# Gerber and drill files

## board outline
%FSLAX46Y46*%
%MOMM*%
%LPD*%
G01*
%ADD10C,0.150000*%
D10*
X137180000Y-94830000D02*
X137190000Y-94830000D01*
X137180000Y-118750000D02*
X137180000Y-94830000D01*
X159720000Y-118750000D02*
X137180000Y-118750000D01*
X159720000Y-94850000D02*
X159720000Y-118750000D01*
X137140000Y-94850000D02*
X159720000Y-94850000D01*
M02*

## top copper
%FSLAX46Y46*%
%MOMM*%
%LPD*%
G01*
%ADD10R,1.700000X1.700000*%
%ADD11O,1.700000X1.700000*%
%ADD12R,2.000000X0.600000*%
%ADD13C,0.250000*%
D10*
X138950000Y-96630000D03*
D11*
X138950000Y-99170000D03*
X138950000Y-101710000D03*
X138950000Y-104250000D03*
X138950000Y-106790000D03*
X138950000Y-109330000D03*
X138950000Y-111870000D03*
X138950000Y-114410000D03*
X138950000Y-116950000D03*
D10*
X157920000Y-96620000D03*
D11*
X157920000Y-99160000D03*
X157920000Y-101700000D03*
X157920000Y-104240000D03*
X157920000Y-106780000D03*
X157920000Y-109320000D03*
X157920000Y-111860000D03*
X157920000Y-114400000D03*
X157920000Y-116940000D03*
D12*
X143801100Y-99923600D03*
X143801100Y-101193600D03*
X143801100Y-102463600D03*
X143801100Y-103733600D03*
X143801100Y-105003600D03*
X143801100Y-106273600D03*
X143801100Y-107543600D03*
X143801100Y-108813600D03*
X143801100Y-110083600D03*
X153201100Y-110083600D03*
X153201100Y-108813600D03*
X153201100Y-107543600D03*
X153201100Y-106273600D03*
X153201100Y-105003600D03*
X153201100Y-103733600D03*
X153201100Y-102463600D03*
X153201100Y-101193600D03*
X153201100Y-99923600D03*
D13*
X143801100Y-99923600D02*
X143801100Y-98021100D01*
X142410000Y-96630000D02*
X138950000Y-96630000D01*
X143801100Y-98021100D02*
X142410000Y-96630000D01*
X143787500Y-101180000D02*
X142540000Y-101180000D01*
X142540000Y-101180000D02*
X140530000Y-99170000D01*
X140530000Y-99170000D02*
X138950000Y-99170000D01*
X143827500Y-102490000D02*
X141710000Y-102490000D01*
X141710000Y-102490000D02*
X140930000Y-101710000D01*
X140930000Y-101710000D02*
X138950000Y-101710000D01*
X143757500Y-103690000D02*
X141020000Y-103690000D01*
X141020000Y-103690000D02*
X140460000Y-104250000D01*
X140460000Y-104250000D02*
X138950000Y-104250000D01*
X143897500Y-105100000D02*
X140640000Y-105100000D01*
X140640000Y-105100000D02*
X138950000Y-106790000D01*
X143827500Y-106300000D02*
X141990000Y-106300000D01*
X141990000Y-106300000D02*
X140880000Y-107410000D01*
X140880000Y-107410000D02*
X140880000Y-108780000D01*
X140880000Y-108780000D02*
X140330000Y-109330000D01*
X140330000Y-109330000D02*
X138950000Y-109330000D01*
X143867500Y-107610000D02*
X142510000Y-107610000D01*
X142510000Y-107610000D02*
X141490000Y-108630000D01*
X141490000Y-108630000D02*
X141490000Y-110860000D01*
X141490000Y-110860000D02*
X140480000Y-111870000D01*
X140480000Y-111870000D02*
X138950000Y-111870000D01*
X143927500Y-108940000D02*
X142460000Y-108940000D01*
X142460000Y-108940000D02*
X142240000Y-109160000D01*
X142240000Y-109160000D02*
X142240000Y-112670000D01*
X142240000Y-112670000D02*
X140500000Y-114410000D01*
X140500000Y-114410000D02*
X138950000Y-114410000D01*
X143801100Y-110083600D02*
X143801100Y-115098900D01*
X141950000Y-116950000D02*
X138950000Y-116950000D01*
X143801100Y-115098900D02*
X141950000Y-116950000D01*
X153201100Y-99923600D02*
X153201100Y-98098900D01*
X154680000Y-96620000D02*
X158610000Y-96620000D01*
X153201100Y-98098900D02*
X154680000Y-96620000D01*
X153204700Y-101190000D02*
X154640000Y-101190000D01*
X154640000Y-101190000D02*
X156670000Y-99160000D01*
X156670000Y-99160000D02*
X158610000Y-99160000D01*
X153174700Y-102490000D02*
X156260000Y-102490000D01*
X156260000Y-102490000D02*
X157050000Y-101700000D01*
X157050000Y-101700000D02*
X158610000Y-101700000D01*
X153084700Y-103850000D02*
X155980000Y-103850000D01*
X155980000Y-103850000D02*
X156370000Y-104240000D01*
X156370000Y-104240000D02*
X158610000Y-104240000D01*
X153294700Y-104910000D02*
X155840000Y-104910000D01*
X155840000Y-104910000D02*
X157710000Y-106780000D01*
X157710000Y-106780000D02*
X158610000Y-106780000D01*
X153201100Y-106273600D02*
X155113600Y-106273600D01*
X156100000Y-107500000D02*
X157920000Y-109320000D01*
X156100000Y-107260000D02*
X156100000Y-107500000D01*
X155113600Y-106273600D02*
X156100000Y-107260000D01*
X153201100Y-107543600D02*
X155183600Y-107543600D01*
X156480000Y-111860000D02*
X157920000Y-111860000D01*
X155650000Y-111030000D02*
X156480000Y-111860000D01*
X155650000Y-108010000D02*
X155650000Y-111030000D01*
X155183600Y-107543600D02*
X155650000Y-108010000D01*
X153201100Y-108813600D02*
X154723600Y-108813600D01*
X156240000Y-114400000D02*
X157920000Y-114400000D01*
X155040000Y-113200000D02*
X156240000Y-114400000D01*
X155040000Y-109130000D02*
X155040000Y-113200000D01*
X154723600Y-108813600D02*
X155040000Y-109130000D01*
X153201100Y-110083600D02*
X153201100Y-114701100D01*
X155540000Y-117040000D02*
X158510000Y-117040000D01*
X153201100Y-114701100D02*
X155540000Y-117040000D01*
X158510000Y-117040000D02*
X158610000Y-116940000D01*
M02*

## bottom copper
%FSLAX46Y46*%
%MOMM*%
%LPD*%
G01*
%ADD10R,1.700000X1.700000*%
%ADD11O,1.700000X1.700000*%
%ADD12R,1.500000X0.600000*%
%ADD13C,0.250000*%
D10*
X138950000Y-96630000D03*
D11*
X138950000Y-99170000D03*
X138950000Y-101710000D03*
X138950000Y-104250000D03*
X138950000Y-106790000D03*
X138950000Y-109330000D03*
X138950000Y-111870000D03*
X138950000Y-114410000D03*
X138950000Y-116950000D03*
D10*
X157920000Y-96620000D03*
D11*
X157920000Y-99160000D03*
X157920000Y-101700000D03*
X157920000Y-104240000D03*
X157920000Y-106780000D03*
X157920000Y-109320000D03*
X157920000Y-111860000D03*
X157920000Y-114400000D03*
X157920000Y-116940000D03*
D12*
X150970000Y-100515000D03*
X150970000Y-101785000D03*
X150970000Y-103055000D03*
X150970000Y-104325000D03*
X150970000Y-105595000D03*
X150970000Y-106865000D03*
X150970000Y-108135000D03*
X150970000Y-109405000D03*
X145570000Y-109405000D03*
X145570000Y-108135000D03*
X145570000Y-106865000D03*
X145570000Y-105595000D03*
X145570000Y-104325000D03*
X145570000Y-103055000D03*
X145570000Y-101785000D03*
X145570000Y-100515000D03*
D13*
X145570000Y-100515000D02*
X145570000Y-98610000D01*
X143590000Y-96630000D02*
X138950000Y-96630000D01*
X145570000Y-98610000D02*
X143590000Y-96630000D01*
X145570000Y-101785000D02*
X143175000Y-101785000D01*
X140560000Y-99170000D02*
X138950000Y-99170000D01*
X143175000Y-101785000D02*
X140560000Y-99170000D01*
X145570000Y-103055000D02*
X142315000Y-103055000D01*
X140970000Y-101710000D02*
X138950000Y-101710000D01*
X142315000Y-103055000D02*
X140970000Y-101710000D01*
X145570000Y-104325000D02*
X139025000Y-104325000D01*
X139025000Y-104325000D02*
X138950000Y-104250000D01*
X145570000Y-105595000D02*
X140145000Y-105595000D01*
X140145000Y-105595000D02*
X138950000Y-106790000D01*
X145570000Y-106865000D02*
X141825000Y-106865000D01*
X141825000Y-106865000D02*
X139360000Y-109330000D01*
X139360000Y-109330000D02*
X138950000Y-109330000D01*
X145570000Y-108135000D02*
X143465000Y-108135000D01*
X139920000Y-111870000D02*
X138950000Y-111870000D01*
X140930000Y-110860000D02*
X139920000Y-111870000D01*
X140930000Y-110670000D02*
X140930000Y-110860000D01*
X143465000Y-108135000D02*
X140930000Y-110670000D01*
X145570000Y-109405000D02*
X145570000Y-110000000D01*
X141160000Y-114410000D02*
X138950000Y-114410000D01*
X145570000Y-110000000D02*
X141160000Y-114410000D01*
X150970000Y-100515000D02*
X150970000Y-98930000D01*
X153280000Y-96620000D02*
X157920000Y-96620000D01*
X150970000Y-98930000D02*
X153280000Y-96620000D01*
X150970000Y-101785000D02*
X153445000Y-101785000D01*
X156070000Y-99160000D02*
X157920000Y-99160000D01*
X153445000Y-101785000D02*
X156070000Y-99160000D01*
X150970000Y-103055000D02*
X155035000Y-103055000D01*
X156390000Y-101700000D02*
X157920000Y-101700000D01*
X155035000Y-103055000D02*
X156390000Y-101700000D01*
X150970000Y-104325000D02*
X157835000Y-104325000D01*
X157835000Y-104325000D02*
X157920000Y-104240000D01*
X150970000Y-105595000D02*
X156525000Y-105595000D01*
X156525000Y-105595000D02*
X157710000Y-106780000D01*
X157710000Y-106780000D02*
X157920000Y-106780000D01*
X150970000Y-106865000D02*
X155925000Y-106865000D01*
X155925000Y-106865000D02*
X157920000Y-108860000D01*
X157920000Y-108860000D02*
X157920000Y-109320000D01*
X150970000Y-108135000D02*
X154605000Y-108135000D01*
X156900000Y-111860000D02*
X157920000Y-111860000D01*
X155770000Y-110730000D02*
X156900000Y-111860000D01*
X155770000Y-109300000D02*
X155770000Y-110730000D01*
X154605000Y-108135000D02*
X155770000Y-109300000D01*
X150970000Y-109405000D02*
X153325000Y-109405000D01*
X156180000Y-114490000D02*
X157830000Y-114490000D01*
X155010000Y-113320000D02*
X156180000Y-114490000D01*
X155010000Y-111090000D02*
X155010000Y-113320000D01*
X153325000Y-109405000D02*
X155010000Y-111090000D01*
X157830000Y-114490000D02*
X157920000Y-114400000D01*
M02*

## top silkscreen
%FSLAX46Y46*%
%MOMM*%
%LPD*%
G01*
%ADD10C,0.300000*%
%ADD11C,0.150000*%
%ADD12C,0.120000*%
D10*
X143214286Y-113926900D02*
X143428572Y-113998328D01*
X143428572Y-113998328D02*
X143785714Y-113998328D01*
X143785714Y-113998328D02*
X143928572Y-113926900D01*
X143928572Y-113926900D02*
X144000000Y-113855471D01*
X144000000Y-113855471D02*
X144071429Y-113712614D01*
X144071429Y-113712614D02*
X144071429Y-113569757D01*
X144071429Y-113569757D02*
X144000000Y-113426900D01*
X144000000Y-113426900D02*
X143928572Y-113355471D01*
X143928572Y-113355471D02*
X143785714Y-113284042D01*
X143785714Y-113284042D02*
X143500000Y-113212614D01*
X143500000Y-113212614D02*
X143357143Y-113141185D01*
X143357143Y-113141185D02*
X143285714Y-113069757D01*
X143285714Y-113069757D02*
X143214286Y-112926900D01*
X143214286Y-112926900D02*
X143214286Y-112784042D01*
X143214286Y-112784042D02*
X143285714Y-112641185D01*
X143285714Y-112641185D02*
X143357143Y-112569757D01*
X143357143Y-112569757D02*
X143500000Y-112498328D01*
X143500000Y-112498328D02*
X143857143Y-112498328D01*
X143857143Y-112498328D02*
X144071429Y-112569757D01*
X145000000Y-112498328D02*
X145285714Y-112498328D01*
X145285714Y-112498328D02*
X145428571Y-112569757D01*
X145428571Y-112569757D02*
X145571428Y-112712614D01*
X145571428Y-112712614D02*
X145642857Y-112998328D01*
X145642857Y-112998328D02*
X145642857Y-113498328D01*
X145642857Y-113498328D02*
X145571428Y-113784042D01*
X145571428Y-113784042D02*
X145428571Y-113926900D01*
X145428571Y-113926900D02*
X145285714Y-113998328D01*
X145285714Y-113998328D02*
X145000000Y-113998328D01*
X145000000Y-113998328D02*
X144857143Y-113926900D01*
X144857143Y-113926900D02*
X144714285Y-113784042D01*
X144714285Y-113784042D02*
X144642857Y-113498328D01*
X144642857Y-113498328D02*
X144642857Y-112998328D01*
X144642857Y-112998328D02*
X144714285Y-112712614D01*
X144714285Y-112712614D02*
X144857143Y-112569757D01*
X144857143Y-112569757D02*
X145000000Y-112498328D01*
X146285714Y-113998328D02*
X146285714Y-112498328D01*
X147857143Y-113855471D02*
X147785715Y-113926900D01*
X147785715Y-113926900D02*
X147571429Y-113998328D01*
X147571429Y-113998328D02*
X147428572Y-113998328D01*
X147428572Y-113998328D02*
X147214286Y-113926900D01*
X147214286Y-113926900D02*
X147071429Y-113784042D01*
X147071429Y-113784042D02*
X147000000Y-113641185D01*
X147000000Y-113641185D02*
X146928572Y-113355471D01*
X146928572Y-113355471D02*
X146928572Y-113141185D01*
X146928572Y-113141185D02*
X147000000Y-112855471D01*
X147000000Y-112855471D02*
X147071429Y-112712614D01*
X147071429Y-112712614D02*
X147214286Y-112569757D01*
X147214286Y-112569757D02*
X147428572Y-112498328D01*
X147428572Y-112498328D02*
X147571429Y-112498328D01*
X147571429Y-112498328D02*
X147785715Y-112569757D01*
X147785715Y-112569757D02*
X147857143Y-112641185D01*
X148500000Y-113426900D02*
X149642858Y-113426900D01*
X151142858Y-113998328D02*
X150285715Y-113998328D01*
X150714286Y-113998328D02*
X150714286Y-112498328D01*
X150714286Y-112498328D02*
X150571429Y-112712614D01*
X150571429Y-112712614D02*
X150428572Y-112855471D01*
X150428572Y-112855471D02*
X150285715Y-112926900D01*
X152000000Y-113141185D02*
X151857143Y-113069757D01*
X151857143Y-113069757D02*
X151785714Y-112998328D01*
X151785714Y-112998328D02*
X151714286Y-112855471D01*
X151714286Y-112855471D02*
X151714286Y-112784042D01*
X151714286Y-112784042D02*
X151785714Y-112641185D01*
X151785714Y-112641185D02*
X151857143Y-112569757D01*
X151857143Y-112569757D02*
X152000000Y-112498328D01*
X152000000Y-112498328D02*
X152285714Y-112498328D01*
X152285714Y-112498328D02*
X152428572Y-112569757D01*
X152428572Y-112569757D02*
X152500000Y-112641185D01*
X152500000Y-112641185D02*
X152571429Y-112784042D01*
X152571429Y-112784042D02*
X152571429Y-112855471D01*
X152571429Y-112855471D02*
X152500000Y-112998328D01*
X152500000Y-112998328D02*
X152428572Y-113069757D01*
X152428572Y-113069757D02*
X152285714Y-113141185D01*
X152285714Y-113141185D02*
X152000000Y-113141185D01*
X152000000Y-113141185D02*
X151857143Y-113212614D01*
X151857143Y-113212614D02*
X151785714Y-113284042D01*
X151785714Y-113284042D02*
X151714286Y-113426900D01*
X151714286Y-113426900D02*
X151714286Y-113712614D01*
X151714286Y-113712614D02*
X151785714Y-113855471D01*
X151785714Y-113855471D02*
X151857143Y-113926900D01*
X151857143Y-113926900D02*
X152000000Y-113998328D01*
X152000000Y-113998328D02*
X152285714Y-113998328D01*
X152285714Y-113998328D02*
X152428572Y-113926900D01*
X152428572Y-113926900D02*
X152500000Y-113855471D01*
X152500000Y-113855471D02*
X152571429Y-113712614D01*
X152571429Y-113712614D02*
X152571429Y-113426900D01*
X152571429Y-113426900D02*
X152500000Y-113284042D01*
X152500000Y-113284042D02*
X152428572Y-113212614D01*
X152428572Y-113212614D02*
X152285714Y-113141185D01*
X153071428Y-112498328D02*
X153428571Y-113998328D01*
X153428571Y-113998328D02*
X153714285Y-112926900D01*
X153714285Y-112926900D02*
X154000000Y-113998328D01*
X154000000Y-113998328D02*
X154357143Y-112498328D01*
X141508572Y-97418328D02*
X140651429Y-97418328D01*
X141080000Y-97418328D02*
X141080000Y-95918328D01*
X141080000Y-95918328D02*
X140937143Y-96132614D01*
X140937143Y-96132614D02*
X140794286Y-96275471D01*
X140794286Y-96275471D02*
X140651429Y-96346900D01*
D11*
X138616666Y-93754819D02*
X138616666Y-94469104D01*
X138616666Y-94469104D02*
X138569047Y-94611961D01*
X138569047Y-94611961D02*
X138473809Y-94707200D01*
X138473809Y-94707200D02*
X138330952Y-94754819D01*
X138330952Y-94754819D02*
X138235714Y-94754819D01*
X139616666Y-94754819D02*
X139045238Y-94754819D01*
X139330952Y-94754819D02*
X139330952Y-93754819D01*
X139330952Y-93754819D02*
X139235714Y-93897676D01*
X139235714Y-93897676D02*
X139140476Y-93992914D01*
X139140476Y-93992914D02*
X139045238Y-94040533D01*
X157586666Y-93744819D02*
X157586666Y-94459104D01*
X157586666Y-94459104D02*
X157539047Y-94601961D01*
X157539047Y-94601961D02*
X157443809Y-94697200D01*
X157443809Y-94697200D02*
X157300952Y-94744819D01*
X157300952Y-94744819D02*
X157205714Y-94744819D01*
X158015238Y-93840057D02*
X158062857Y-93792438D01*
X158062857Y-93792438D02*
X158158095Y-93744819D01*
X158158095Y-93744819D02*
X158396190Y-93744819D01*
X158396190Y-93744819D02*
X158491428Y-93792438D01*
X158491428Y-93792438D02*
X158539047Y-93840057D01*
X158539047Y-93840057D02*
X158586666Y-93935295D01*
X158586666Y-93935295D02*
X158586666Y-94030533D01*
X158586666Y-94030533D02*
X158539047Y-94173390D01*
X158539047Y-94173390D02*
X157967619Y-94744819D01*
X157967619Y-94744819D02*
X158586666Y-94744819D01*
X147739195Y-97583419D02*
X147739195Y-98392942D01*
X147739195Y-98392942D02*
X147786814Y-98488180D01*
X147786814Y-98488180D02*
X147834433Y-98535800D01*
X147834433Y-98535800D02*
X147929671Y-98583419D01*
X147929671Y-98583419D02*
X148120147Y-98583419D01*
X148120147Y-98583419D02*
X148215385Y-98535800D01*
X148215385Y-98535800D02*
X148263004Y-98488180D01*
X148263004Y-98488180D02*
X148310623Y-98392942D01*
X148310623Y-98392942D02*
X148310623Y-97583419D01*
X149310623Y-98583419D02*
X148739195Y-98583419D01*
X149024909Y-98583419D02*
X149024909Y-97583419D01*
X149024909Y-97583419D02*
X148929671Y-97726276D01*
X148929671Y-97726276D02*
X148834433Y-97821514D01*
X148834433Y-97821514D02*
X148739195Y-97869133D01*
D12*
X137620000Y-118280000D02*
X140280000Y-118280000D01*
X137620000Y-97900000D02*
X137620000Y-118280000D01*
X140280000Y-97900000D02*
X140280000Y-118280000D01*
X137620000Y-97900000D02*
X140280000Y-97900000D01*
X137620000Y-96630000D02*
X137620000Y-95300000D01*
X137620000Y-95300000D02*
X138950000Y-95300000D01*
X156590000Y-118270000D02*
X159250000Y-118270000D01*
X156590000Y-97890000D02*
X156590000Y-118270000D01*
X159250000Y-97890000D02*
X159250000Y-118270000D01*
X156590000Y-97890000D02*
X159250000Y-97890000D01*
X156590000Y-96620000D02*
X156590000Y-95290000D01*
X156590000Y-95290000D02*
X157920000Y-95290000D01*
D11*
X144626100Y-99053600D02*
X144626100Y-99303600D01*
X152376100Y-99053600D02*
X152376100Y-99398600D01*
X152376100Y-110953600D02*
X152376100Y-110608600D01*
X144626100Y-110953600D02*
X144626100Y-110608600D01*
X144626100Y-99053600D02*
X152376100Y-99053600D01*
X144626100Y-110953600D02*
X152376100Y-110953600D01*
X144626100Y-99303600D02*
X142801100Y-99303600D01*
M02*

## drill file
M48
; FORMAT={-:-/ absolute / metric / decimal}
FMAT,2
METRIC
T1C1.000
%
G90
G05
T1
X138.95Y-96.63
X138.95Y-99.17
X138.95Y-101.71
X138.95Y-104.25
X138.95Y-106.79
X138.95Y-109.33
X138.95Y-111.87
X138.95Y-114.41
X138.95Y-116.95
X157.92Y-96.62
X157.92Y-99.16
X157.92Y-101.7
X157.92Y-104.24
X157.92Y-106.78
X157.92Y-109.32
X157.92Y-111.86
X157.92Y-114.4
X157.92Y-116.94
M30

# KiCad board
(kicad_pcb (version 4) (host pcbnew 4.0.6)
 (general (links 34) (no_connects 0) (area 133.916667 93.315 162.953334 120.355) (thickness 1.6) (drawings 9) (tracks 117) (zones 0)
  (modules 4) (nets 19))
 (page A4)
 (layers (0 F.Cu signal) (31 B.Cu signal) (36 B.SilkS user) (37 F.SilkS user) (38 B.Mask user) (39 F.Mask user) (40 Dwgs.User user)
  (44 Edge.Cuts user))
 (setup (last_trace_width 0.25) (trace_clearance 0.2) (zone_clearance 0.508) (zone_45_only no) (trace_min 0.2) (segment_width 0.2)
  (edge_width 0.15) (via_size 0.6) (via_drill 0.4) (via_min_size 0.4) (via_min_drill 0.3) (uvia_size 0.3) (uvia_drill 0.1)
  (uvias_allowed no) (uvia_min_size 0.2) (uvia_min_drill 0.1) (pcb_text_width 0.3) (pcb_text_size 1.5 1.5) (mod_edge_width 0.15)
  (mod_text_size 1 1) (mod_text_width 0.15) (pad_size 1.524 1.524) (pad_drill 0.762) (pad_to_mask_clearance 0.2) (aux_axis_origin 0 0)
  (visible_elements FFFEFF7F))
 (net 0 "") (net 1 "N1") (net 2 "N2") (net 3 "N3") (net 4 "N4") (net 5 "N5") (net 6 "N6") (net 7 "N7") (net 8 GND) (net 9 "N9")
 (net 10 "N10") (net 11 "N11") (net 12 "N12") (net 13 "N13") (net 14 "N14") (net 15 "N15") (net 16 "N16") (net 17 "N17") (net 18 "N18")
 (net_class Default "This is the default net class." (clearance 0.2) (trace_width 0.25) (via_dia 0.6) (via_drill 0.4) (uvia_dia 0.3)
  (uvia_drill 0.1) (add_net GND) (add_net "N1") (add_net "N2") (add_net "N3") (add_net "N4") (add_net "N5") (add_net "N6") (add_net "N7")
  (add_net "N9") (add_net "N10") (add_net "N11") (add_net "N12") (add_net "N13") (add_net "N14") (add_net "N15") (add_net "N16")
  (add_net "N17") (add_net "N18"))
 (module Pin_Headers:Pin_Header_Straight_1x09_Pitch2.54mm (layer F.Cu) (at 138.95 96.63)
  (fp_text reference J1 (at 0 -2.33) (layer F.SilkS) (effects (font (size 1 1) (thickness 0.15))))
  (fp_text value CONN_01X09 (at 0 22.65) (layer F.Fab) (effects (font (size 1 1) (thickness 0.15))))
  (fp_line (start -1.33 21.65) (end 1.33 21.65) (layer F.SilkS) (width 0.12))
  (fp_line (start -1.33 1.27) (end -1.33 21.65) (layer F.SilkS) (width 0.12))
  (fp_line (start 1.33 1.27) (end 1.33 21.65) (layer F.SilkS) (width 0.12))
  (fp_line (start -1.33 1.27) (end 1.33 1.27) (layer F.SilkS) (width 0.12))
  (fp_line (start -1.33 0) (end -1.33 -1.33) (layer F.SilkS) (width 0.12))
  (fp_line (start -1.33 -1.33) (end 0 -1.33) (layer F.SilkS) (width 0.12))
  (pad 1 thru_hole rect (at 0 0) (size 1.7 1.7) (drill 1) (layers *.Cu *.Mask) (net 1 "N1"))
  (pad 2 thru_hole oval (at 0 2.54) (size 1.7 1.7) (drill 1) (layers *.Cu *.Mask) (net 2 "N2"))
  (pad 3 thru_hole oval (at 0 5.08) (size 1.7 1.7) (drill 1) (layers *.Cu *.Mask) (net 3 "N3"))
  (pad 4 thru_hole oval (at 0 7.62) (size 1.7 1.7) (drill 1) (layers *.Cu *.Mask) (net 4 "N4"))
  (pad 5 thru_hole oval (at 0 10.16) (size 1.7 1.7) (drill 1) (layers *.Cu *.Mask) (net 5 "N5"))
  (pad 6 thru_hole oval (at 0 12.7) (size 1.7 1.7) (drill 1) (layers *.Cu *.Mask) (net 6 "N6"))
  (pad 7 thru_hole oval (at 0 15.24) (size 1.7 1.7) (drill 1) (layers *.Cu *.Mask) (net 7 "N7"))
  (pad 8 thru_hole oval (at 0 17.78) (size 1.7 1.7) (drill 1) (layers *.Cu *.Mask) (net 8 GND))
  (pad 9 thru_hole oval (at 0 20.32) (size 1.7 1.7) (drill 1) (layers *.Cu *.Mask) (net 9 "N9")))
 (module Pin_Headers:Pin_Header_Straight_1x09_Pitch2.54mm (layer F.Cu) (at 157.92 96.62)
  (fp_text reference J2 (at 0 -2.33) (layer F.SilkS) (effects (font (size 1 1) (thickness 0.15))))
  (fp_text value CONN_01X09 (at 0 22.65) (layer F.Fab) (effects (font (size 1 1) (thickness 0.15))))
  (fp_line (start -1.33 21.65) (end 1.33 21.65) (layer F.SilkS) (width 0.12))
  (fp_line (start -1.33 1.27) (end -1.33 21.65) (layer F.SilkS) (width 0.12))
  (fp_line (start 1.33 1.27) (end 1.33 21.65) (layer F.SilkS) (width 0.12))
  (fp_line (start -1.33 1.27) (end 1.33 1.27) (layer F.SilkS) (width 0.12))
  (fp_line (start -1.33 0) (end -1.33 -1.33) (layer F.SilkS) (width 0.12))
  (fp_line (start -1.33 -1.33) (end 0 -1.33) (layer F.SilkS) (width 0.12))
  (pad 1 thru_hole rect (at 0 0) (size 1.7 1.7) (drill 1) (layers *.Cu *.Mask) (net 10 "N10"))
  (pad 2 thru_hole oval (at 0 2.54) (size 1.7 1.7) (drill 1) (layers *.Cu *.Mask) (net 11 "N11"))
  (pad 3 thru_hole oval (at 0 5.08) (size 1.7 1.7) (drill 1) (layers *.Cu *.Mask) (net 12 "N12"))
  (pad 4 thru_hole oval (at 0 7.62) (size 1.7 1.7) (drill 1) (layers *.Cu *.Mask) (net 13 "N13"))
  (pad 5 thru_hole oval (at 0 10.16) (size 1.7 1.7) (drill 1) (layers *.Cu *.Mask) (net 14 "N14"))
  (pad 6 thru_hole oval (at 0 12.7) (size 1.7 1.7) (drill 1) (layers *.Cu *.Mask) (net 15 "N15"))
  (pad 7 thru_hole oval (at 0 15.24) (size 1.7 1.7) (drill 1) (layers *.Cu *.Mask) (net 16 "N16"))
  (pad 8 thru_hole oval (at 0 17.78) (size 1.7 1.7) (drill 1) (layers *.Cu *.Mask) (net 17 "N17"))
  (pad 9 thru_hole oval (at 0 20.32) (size 1.7 1.7) (drill 1) (layers *.Cu *.Mask) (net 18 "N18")))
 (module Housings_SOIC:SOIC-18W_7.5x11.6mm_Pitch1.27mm (layer F.Cu) (at 148.5011 105.0036)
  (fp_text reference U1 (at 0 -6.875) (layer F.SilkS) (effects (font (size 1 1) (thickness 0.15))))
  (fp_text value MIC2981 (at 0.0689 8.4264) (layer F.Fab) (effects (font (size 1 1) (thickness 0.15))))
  (fp_line (start -3.875 -5.95) (end -3.875 -5.7) (layer F.SilkS) (width 0.15))
  (fp_line (start 3.875 -5.95) (end 3.875 -5.605) (layer F.SilkS) (width 0.15))
  (fp_line (start 3.875 5.95) (end 3.875 5.605) (layer F.SilkS) (width 0.15))
  (fp_line (start -3.875 5.95) (end -3.875 5.605) (layer F.SilkS) (width 0.15))
  (fp_line (start -3.875 -5.95) (end 3.875 -5.95) (layer F.SilkS) (width 0.15))
  (fp_line (start -3.875 5.95) (end 3.875 5.95) (layer F.SilkS) (width 0.15))
  (fp_line (start -3.875 -5.7) (end -5.7 -5.7) (layer F.SilkS) (width 0.15))
  (pad 1 smd rect (at -4.7 -5.08) (size 2 0.6) (layers F.Cu F.Mask) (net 1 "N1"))
  (pad 2 smd rect (at -4.7 -3.81) (size 2 0.6) (layers F.Cu F.Mask) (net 2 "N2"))
  (pad 3 smd rect (at -4.7 -2.54) (size 2 0.6) (layers F.Cu F.Mask) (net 3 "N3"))
  (pad 4 smd rect (at -4.7 -1.27) (size 2 0.6) (layers F.Cu F.Mask) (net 4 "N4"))
  (pad 5 smd rect (at -4.7 0) (size 2 0.6) (layers F.Cu F.Mask) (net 5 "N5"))
  (pad 6 smd rect (at -4.7 1.27) (size 2 0.6) (layers F.Cu F.Mask) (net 6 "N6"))
  (pad 7 smd rect (at -4.7 2.54) (size 2 0.6) (layers F.Cu F.Mask) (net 7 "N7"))
  (pad 8 smd rect (at -4.7 3.81) (size 2 0.6) (layers F.Cu F.Mask) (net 8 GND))
  (pad 9 smd rect (at -4.7 5.08) (size 2 0.6) (layers F.Cu F.Mask) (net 9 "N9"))
  (pad 10 smd rect (at 4.7 5.08) (size 2 0.6) (layers F.Cu F.Mask) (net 18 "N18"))
  (pad 11 smd rect (at 4.7 3.81) (size 2 0.6) (layers F.Cu F.Mask) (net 17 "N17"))
  (pad 12 smd rect (at 4.7 2.54) (size 2 0.6) (layers F.Cu F.Mask) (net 16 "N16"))
  (pad 13 smd rect (at 4.7 1.27) (size 2 0.6) (layers F.Cu F.Mask) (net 15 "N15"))
  (pad 14 smd rect (at 4.7 0) (size 2 0.6) (layers F.Cu F.Mask) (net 14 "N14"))
  (pad 15 smd rect (at 4.7 -1.27) (size 2 0.6) (layers F.Cu F.Mask) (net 13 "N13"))
  (pad 16 smd rect (at 4.7 -2.54) (size 2 0.6) (layers F.Cu F.Mask) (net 12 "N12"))
  (pad 17 smd rect (at 4.7 -3.81) (size 2 0.6) (layers F.Cu F.Mask) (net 11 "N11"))
  (pad 18 smd rect (at 4.7 -5.08) (size 2 0.6) (layers F.Cu F.Mask) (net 10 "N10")))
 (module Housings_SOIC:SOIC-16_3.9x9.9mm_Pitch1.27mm (layer B.Cu) (at 148.27 104.96 180)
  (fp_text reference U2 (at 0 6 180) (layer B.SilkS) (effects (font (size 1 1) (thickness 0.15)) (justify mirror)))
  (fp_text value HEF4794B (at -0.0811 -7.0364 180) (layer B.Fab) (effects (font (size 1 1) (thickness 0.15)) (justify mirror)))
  (pad 1 smd rect (at -2.7 4.445 180) (size 1.5 0.6) (layers B.Cu B.Mask) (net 10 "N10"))
  (pad 2 smd rect (at -2.7 3.175 180) (size 1.5 0.6) (layers B.Cu B.Mask) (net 11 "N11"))
  (pad 3 smd rect (at -2.7 1.905 180) (size 1.5 0.6) (layers B.Cu B.Mask) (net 12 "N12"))
  (pad 4 smd rect (at -2.7 0.635 180) (size 1.5 0.6) (layers B.Cu B.Mask) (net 13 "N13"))
  (pad 5 smd rect (at -2.7 -0.635 180) (size 1.5 0.6) (layers B.Cu B.Mask) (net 14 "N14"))
  (pad 6 smd rect (at -2.7 -1.905 180) (size 1.5 0.6) (layers B.Cu B.Mask) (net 15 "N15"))
  (pad 7 smd rect (at -2.7 -3.175 180) (size 1.5 0.6) (layers B.Cu B.Mask) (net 16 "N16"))
  (pad 8 smd rect (at -2.7 -4.445 180) (size 1.5 0.6) (layers B.Cu B.Mask) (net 17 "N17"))
  (pad 9 smd rect (at 2.7 -4.445 180) (size 1.5 0.6) (layers B.Cu B.Mask) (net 8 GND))
  (pad 10 smd rect (at 2.7 -3.175 180) (size 1.5 0.6) (layers B.Cu B.Mask) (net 7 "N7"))
  (pad 11 smd rect (at 2.7 -1.905 180) (size 1.5 0.6) (layers B.Cu B.Mask) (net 6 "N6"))
  (pad 12 smd rect (at 2.7 -0.635 180) (size 1.5 0.6) (layers B.Cu B.Mask) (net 5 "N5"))
  (pad 13 smd rect (at 2.7 0.635 180) (size 1.5 0.6) (layers B.Cu B.Mask) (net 4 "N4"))
  (pad 14 smd rect (at 2.7 1.905 180) (size 1.5 0.6) (layers B.Cu B.Mask) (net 3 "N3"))
  (pad 15 smd rect (at 2.7 3.175 180) (size 1.5 0.6) (layers B.Cu B.Mask) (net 2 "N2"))
  (pad 16 smd rect (at 2.7 4.445 180) (size 1.5 0.6) (layers B.Cu B.Mask) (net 1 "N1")))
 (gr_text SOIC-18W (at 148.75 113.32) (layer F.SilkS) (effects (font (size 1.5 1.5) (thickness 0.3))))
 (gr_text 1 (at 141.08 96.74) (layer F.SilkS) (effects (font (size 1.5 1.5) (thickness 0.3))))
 (gr_line (start 137.18 94.83) (end 137.19 94.83) (angle 90) (layer Edge.Cuts) (width 0.15))
 (gr_line (start 137.18 118.75) (end 137.18 94.83) (angle 90) (layer Edge.Cuts) (width 0.15))
 (gr_line (start 159.72 118.75) (end 137.18 118.75) (angle 90) (layer Edge.Cuts) (width 0.15))
 (gr_line (start 159.72 94.85) (end 159.72 118.75) (angle 90) (layer Edge.Cuts) (width 0.15))
 (gr_line (start 137.14 94.85) (end 159.72 94.85) (angle 90) (layer Edge.Cuts) (width 0.15))
 (segment (start 145.57 100.515) (end 145.57 98.61) (width 0.25) (layer B.Cu) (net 1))
 (segment (start 143.59 96.63) (end 138.95 96.63) (width 0.25) (layer B.Cu) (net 1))
 (segment (start 145.57 98.61) (end 143.59 96.63) (width 0.25) (layer B.Cu) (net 1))
 (segment (start 143.8011 99.9236) (end 143.8011 98.0211) (width 0.25) (layer F.Cu) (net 1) (status 10))
 (segment (start 142.41 96.63) (end 138.95 96.63) (width 0.25) (layer F.Cu) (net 1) (status 20))
 (segment (start 143.8011 98.0211) (end 142.41 96.63) (width 0.25) (layer F.Cu) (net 1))
 (segment (start 145.57 101.785) (end 143.175 101.785) (width 0.25) (layer B.Cu) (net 2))
 (segment (start 140.56 99.17) (end 138.95 99.17) (width 0.25) (layer B.Cu) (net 2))
 (segment (start 143.175 101.785) (end 140.56 99.17) (width 0.25) (layer B.Cu) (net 2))
 (segment (start 143.7875 101.18) (end 142.54 101.18) (width 0.25) (layer F.Cu) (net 2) (status 10))
 (segment (start 142.54 101.18) (end 140.53 99.17) (width 0.25) (layer F.Cu) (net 2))
 (segment (start 140.53 99.17) (end 138.95 99.17) (width 0.25) (layer F.Cu) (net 2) (status 20))
 (segment (start 145.57 103.055) (end 142.315 103.055) (width 0.25) (layer B.Cu) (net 3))
 (segment (start 140.97 101.71) (end 138.95 101.71) (width 0.25) (layer B.Cu) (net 3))
 (segment (start 142.315 103.055) (end 140.97 101.71) (width 0.25) (layer B.Cu) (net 3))
 (segment (start 143.8275 102.49) (end 141.71 102.49) (width 0.25) (layer F.Cu) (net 3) (status 10))
 (segment (start 141.71 102.49) (end 140.93 101.71) (width 0.25) (layer F.Cu) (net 3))
 (segment (start 140.93 101.71) (end 138.95 101.71) (width 0.25) (layer F.Cu) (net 3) (status 20))
 (segment (start 145.57 104.325) (end 139.025 104.325) (width 0.25) (layer B.Cu) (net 4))
 (segment (start 139.025 104.325) (end 138.95 104.25) (width 0.25) (layer B.Cu) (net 4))
 (segment (start 143.7575 103.69) (end 141.02 103.69) (width 0.25) (layer F.Cu) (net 4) (status 10))
 (segment (start 141.02 103.69) (end 140.46 104.25) (width 0.25) (layer F.Cu) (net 4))
 (segment (start 140.46 104.25) (end 138.95 104.25) (width 0.25) (layer F.Cu) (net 4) (status 20))
 (segment (start 145.57 105.595) (end 140.145 105.595) (width 0.25) (layer B.Cu) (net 5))
 (segment (start 140.145 105.595) (end 138.95 106.79) (width 0.25) (layer B.Cu) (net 5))
 (segment (start 143.8975 105.1) (end 140.64 105.1) (width 0.25) (layer F.Cu) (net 5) (status 10))
 (segment (start 140.64 105.1) (end 138.95 106.79) (width 0.25) (layer F.Cu) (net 5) (status 20))
 (segment (start 145.57 106.865) (end 141.825 106.865) (width 0.25) (layer B.Cu) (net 6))
 (segment (start 141.825 106.865) (end 139.36 109.33) (width 0.25) (layer B.Cu) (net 6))
 (segment (start 139.36 109.33) (end 138.95 109.33) (width 0.25) (layer B.Cu) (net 6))
 (segment (start 143.8275 106.3) (end 141.99 106.3) (width 0.25) (layer F.Cu) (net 6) (status 10))
 (segment (start 141.99 106.3) (end 140.88 107.41) (width 0.25) (layer F.Cu) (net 6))
 (segment (start 140.88 107.41) (end 140.88 108.78) (width 0.25) (layer F.Cu) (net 6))
 (segment (start 140.88 108.78) (end 140.33 109.33) (width 0.25) (layer F.Cu) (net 6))
 (segment (start 140.33 109.33) (end 138.95 109.33) (width 0.25) (layer F.Cu) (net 6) (status 20))
 (segment (start 145.57 108.135) (end 143.465 108.135) (width 0.25) (layer B.Cu) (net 7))
 (segment (start 139.92 111.87) (end 138.95 111.87) (width 0.25) (layer B.Cu) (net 7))
 (segment (start 140.93 110.86) (end 139.92 111.87) (width 0.25) (layer B.Cu) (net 7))
 (segment (start 140.93 110.67) (end 140.93 110.86) (width 0.25) (layer B.Cu) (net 7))
 (segment (start 143.465 108.135) (end 140.93 110.67) (width 0.25) (layer B.Cu) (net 7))
 (segment (start 143.8675 107.61) (end 142.51 107.61) (width 0.25) (layer F.Cu) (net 7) (status 10))
 (segment (start 142.51 107.61) (end 141.49 108.63) (width 0.25) (layer F.Cu) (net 7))
 (segment (start 141.49 108.63) (end 141.49 110.86) (width 0.25) (layer F.Cu) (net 7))
 (segment (start 141.49 110.86) (end 140.48 111.87) (width 0.25) (layer F.Cu) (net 7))
 (segment (start 140.48 111.87) (end 138.95 111.87) (width 0.25) (layer F.Cu) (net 7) (status 20))
 (segment (start 145.57 109.405) (end 145.57 110) (width 0.25) (layer B.Cu) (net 8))
 (segment (start 141.16 114.41) (end 138.95 114.41) (width 0.25) (layer B.Cu) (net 8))
 (segment (start 145.57 110) (end 141.16 114.41) (width 0.25) (layer B.Cu) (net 8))
 (segment (start 143.9275 108.94) (end 142.46 108.94) (width 0.25) (layer F.Cu) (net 8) (status 10))
 (segment (start 142.46 108.94) (end 142.24 109.16) (width 0.25) (layer F.Cu) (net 8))
 (segment (start 142.24 109.16) (end 142.24 112.67) (width 0.25) (layer F.Cu) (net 8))
 (segment (start 142.24 112.67) (end 140.5 114.41) (width 0.25) (layer F.Cu) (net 8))
 (segment (start 140.5 114.41) (end 138.95 114.41) (width 0.25) (layer F.Cu) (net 8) (status 20))
 (segment (start 143.8011 110.0836) (end 143.8011 115.0989) (width 0.25) (layer F.Cu) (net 9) (status 10))
 (segment (start 141.95 116.95) (end 138.95 116.95) (width 0.25) (layer F.Cu) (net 9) (status 20))
 (segment (start 143.8011 115.0989) (end 141.95 116.95) (width 0.25) (layer F.Cu) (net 9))
 (segment (start 150.97 100.515) (end 150.97 98.93) (width 0.25) (layer B.Cu) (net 10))
 (segment (start 153.28 96.62) (end 157.92 96.62) (width 0.25) (layer B.Cu) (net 10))
 (segment (start 150.97 98.93) (end 153.28 96.62) (width 0.25) (layer B.Cu) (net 10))
 (segment (start 153.2011 99.9236) (end 153.2011 98.0989) (width 0.25) (layer F.Cu) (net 10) (status 10))
 (segment (start 154.68 96.62) (end 158.61 96.62) (width 0.25) (layer F.Cu) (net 10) (status 20))
 (segment (start 153.2011 98.0989) (end 154.68 96.62) (width 0.25) (layer F.Cu) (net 10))
 (segment (start 150.97 101.785) (end 153.445 101.785) (width 0.25) (layer B.Cu) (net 11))
 (segment (start 156.07 99.16) (end 157.92 99.16) (width 0.25) (layer B.Cu) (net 11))
 (segment (start 153.445 101.785) (end 156.07 99.16) (width 0.25) (layer B.Cu) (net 11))
 (segment (start 153.2047 101.19) (end 154.64 101.19) (width 0.25) (layer F.Cu) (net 11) (status 10))
 (segment (start 154.64 101.19) (end 156.67 99.16) (width 0.25) (layer F.Cu) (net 11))
 (segment (start 156.67 99.16) (end 158.61 99.16) (width 0.25) (layer F.Cu) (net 11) (status 20))
 (segment (start 150.97 103.055) (end 155.035 103.055) (width 0.25) (layer B.Cu) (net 12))
 (segment (start 156.39 101.7) (end 157.92 101.7) (width 0.25) (layer B.Cu) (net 12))
 (segment (start 155.035 103.055) (end 156.39 101.7) (width 0.25) (layer B.Cu) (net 12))
 (segment (start 153.1747 102.49) (end 156.26 102.49) (width 0.25) (layer F.Cu) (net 12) (status 10))
 (segment (start 156.26 102.49) (end 157.05 101.7) (width 0.25) (layer F.Cu) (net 12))
 (segment (start 157.05 101.7) (end 158.61 101.7) (width 0.25) (layer F.Cu) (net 12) (status 20))
 (segment (start 150.97 104.325) (end 157.835 104.325) (width 0.25) (layer B.Cu) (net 13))
 (segment (start 157.835 104.325) (end 157.92 104.24) (width 0.25) (layer B.Cu) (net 13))
 (segment (start 153.0847 103.85) (end 155.98 103.85) (width 0.25) (layer F.Cu) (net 13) (status 10))
 (segment (start 155.98 103.85) (end 156.37 104.24) (width 0.25) (layer F.Cu) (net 13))
 (segment (start 156.37 104.24) (end 158.61 104.24) (width 0.25) (layer F.Cu) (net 13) (status 20))
 (segment (start 150.97 105.595) (end 156.525 105.595) (width 0.25) (layer B.Cu) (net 14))
 (segment (start 156.525 105.595) (end 157.71 106.78) (width 0.25) (layer B.Cu) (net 14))
 (segment (start 157.71 106.78) (end 157.92 106.78) (width 0.25) (layer B.Cu) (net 14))
 (segment (start 153.2947 104.91) (end 155.84 104.91) (width 0.25) (layer F.Cu) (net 14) (status 10))
 (segment (start 155.84 104.91) (end 157.71 106.78) (width 0.25) (layer F.Cu) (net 14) (status 20))
 (segment (start 157.71 106.78) (end 158.61 106.78) (width 0.25) (layer F.Cu) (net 14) (status 30))
 (segment (start 150.97 106.865) (end 155.925 106.865) (width 0.25) (layer B.Cu) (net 15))
 (segment (start 155.925 106.865) (end 157.92 108.86) (width 0.25) (layer B.Cu) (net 15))
 (segment (start 157.92 108.86) (end 157.92 109.32) (width 0.25) (layer B.Cu) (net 15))
 (segment (start 153.2011 106.2736) (end 155.1136 106.2736) (width 0.25) (layer F.Cu) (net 15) (status 10))
 (segment (start 156.1 107.5) (end 157.92 109.32) (width 0.25) (layer F.Cu) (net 15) (status 20))
 (segment (start 156.1 107.26) (end 156.1 107.5) (width 0.25) (layer F.Cu) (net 15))
 (segment (start 155.1136 106.2736) (end 156.1 107.26) (width 0.25) (layer F.Cu) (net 15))
 (segment (start 150.97 108.135) (end 154.605 108.135) (width 0.25) (layer B.Cu) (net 16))
 (segment (start 156.9 111.86) (end 157.92 111.86) (width 0.25) (layer B.Cu) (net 16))
 (segment (start 155.77 110.73) (end 156.9 111.86) (width 0.25) (layer B.Cu) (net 16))
 (segment (start 155.77 109.3) (end 155.77 110.73) (width 0.25) (layer B.Cu) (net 16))
 (segment (start 154.605 108.135) (end 155.77 109.3) (width 0.25) (layer B.Cu) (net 16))
 (segment (start 153.2011 107.5436) (end 155.1836 107.5436) (width 0.25) (layer F.Cu) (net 16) (status 10))
 (segment (start 156.48 111.86) (end 157.92 111.86) (width 0.25) (layer F.Cu) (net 16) (status 20))
 (segment (start 155.65 111.03) (end 156.48 111.86) (width 0.25) (layer F.Cu) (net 16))
 (segment (start 155.65 108.01) (end 155.65 111.03) (width 0.25) (layer F.Cu) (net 16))
 (segment (start 155.1836 107.5436) (end 155.65 108.01) (width 0.25) (layer F.Cu) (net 16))
 (segment (start 150.97 109.405) (end 153.325 109.405) (width 0.25) (layer B.Cu) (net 17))
 (segment (start 156.18 114.49) (end 157.83 114.49) (width 0.25) (layer B.Cu) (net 17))
 (segment (start 155.01 113.32) (end 156.18 114.49) (width 0.25) (layer B.Cu) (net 17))
 (segment (start 155.01 111.09) (end 155.01 113.32) (width 0.25) (layer B.Cu) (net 17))
 (segment (start 153.325 109.405) (end 155.01 111.09) (width 0.25) (layer B.Cu) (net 17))
 (segment (start 157.83 114.49) (end 157.92 114.4) (width 0.25) (layer B.Cu) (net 17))
 (segment (start 153.2011 108.8136) (end 154.7236 108.8136) (width 0.25) (layer F.Cu) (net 17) (status 10))
 (segment (start 156.24 114.4) (end 157.92 114.4) (width 0.25) (layer F.Cu) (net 17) (status 20))
 (segment (start 155.04 113.2) (end 156.24 114.4) (width 0.25) (layer F.Cu) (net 17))
 (segment (start 155.04 109.13) (end 155.04 113.2) (width 0.25) (layer F.Cu) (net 17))
 (segment (start 154.7236 108.8136) (end 155.04 109.13) (width 0.25) (layer F.Cu) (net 17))
 (segment (start 153.2011 110.0836) (end 153.2011 114.7011) (width 0.25) (layer F.Cu) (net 18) (status 10))
 (segment (start 155.54 117.04) (end 158.51 117.04) (width 0.25) (layer F.Cu) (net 18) (status 20))
 (segment (start 153.2011 114.7011) (end 155.54 117.04) (width 0.25) (layer F.Cu) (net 18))
 (segment (start 158.51 117.04) (end 158.61 116.94) (width 0.25) (layer F.Cu) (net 18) (status 30)))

